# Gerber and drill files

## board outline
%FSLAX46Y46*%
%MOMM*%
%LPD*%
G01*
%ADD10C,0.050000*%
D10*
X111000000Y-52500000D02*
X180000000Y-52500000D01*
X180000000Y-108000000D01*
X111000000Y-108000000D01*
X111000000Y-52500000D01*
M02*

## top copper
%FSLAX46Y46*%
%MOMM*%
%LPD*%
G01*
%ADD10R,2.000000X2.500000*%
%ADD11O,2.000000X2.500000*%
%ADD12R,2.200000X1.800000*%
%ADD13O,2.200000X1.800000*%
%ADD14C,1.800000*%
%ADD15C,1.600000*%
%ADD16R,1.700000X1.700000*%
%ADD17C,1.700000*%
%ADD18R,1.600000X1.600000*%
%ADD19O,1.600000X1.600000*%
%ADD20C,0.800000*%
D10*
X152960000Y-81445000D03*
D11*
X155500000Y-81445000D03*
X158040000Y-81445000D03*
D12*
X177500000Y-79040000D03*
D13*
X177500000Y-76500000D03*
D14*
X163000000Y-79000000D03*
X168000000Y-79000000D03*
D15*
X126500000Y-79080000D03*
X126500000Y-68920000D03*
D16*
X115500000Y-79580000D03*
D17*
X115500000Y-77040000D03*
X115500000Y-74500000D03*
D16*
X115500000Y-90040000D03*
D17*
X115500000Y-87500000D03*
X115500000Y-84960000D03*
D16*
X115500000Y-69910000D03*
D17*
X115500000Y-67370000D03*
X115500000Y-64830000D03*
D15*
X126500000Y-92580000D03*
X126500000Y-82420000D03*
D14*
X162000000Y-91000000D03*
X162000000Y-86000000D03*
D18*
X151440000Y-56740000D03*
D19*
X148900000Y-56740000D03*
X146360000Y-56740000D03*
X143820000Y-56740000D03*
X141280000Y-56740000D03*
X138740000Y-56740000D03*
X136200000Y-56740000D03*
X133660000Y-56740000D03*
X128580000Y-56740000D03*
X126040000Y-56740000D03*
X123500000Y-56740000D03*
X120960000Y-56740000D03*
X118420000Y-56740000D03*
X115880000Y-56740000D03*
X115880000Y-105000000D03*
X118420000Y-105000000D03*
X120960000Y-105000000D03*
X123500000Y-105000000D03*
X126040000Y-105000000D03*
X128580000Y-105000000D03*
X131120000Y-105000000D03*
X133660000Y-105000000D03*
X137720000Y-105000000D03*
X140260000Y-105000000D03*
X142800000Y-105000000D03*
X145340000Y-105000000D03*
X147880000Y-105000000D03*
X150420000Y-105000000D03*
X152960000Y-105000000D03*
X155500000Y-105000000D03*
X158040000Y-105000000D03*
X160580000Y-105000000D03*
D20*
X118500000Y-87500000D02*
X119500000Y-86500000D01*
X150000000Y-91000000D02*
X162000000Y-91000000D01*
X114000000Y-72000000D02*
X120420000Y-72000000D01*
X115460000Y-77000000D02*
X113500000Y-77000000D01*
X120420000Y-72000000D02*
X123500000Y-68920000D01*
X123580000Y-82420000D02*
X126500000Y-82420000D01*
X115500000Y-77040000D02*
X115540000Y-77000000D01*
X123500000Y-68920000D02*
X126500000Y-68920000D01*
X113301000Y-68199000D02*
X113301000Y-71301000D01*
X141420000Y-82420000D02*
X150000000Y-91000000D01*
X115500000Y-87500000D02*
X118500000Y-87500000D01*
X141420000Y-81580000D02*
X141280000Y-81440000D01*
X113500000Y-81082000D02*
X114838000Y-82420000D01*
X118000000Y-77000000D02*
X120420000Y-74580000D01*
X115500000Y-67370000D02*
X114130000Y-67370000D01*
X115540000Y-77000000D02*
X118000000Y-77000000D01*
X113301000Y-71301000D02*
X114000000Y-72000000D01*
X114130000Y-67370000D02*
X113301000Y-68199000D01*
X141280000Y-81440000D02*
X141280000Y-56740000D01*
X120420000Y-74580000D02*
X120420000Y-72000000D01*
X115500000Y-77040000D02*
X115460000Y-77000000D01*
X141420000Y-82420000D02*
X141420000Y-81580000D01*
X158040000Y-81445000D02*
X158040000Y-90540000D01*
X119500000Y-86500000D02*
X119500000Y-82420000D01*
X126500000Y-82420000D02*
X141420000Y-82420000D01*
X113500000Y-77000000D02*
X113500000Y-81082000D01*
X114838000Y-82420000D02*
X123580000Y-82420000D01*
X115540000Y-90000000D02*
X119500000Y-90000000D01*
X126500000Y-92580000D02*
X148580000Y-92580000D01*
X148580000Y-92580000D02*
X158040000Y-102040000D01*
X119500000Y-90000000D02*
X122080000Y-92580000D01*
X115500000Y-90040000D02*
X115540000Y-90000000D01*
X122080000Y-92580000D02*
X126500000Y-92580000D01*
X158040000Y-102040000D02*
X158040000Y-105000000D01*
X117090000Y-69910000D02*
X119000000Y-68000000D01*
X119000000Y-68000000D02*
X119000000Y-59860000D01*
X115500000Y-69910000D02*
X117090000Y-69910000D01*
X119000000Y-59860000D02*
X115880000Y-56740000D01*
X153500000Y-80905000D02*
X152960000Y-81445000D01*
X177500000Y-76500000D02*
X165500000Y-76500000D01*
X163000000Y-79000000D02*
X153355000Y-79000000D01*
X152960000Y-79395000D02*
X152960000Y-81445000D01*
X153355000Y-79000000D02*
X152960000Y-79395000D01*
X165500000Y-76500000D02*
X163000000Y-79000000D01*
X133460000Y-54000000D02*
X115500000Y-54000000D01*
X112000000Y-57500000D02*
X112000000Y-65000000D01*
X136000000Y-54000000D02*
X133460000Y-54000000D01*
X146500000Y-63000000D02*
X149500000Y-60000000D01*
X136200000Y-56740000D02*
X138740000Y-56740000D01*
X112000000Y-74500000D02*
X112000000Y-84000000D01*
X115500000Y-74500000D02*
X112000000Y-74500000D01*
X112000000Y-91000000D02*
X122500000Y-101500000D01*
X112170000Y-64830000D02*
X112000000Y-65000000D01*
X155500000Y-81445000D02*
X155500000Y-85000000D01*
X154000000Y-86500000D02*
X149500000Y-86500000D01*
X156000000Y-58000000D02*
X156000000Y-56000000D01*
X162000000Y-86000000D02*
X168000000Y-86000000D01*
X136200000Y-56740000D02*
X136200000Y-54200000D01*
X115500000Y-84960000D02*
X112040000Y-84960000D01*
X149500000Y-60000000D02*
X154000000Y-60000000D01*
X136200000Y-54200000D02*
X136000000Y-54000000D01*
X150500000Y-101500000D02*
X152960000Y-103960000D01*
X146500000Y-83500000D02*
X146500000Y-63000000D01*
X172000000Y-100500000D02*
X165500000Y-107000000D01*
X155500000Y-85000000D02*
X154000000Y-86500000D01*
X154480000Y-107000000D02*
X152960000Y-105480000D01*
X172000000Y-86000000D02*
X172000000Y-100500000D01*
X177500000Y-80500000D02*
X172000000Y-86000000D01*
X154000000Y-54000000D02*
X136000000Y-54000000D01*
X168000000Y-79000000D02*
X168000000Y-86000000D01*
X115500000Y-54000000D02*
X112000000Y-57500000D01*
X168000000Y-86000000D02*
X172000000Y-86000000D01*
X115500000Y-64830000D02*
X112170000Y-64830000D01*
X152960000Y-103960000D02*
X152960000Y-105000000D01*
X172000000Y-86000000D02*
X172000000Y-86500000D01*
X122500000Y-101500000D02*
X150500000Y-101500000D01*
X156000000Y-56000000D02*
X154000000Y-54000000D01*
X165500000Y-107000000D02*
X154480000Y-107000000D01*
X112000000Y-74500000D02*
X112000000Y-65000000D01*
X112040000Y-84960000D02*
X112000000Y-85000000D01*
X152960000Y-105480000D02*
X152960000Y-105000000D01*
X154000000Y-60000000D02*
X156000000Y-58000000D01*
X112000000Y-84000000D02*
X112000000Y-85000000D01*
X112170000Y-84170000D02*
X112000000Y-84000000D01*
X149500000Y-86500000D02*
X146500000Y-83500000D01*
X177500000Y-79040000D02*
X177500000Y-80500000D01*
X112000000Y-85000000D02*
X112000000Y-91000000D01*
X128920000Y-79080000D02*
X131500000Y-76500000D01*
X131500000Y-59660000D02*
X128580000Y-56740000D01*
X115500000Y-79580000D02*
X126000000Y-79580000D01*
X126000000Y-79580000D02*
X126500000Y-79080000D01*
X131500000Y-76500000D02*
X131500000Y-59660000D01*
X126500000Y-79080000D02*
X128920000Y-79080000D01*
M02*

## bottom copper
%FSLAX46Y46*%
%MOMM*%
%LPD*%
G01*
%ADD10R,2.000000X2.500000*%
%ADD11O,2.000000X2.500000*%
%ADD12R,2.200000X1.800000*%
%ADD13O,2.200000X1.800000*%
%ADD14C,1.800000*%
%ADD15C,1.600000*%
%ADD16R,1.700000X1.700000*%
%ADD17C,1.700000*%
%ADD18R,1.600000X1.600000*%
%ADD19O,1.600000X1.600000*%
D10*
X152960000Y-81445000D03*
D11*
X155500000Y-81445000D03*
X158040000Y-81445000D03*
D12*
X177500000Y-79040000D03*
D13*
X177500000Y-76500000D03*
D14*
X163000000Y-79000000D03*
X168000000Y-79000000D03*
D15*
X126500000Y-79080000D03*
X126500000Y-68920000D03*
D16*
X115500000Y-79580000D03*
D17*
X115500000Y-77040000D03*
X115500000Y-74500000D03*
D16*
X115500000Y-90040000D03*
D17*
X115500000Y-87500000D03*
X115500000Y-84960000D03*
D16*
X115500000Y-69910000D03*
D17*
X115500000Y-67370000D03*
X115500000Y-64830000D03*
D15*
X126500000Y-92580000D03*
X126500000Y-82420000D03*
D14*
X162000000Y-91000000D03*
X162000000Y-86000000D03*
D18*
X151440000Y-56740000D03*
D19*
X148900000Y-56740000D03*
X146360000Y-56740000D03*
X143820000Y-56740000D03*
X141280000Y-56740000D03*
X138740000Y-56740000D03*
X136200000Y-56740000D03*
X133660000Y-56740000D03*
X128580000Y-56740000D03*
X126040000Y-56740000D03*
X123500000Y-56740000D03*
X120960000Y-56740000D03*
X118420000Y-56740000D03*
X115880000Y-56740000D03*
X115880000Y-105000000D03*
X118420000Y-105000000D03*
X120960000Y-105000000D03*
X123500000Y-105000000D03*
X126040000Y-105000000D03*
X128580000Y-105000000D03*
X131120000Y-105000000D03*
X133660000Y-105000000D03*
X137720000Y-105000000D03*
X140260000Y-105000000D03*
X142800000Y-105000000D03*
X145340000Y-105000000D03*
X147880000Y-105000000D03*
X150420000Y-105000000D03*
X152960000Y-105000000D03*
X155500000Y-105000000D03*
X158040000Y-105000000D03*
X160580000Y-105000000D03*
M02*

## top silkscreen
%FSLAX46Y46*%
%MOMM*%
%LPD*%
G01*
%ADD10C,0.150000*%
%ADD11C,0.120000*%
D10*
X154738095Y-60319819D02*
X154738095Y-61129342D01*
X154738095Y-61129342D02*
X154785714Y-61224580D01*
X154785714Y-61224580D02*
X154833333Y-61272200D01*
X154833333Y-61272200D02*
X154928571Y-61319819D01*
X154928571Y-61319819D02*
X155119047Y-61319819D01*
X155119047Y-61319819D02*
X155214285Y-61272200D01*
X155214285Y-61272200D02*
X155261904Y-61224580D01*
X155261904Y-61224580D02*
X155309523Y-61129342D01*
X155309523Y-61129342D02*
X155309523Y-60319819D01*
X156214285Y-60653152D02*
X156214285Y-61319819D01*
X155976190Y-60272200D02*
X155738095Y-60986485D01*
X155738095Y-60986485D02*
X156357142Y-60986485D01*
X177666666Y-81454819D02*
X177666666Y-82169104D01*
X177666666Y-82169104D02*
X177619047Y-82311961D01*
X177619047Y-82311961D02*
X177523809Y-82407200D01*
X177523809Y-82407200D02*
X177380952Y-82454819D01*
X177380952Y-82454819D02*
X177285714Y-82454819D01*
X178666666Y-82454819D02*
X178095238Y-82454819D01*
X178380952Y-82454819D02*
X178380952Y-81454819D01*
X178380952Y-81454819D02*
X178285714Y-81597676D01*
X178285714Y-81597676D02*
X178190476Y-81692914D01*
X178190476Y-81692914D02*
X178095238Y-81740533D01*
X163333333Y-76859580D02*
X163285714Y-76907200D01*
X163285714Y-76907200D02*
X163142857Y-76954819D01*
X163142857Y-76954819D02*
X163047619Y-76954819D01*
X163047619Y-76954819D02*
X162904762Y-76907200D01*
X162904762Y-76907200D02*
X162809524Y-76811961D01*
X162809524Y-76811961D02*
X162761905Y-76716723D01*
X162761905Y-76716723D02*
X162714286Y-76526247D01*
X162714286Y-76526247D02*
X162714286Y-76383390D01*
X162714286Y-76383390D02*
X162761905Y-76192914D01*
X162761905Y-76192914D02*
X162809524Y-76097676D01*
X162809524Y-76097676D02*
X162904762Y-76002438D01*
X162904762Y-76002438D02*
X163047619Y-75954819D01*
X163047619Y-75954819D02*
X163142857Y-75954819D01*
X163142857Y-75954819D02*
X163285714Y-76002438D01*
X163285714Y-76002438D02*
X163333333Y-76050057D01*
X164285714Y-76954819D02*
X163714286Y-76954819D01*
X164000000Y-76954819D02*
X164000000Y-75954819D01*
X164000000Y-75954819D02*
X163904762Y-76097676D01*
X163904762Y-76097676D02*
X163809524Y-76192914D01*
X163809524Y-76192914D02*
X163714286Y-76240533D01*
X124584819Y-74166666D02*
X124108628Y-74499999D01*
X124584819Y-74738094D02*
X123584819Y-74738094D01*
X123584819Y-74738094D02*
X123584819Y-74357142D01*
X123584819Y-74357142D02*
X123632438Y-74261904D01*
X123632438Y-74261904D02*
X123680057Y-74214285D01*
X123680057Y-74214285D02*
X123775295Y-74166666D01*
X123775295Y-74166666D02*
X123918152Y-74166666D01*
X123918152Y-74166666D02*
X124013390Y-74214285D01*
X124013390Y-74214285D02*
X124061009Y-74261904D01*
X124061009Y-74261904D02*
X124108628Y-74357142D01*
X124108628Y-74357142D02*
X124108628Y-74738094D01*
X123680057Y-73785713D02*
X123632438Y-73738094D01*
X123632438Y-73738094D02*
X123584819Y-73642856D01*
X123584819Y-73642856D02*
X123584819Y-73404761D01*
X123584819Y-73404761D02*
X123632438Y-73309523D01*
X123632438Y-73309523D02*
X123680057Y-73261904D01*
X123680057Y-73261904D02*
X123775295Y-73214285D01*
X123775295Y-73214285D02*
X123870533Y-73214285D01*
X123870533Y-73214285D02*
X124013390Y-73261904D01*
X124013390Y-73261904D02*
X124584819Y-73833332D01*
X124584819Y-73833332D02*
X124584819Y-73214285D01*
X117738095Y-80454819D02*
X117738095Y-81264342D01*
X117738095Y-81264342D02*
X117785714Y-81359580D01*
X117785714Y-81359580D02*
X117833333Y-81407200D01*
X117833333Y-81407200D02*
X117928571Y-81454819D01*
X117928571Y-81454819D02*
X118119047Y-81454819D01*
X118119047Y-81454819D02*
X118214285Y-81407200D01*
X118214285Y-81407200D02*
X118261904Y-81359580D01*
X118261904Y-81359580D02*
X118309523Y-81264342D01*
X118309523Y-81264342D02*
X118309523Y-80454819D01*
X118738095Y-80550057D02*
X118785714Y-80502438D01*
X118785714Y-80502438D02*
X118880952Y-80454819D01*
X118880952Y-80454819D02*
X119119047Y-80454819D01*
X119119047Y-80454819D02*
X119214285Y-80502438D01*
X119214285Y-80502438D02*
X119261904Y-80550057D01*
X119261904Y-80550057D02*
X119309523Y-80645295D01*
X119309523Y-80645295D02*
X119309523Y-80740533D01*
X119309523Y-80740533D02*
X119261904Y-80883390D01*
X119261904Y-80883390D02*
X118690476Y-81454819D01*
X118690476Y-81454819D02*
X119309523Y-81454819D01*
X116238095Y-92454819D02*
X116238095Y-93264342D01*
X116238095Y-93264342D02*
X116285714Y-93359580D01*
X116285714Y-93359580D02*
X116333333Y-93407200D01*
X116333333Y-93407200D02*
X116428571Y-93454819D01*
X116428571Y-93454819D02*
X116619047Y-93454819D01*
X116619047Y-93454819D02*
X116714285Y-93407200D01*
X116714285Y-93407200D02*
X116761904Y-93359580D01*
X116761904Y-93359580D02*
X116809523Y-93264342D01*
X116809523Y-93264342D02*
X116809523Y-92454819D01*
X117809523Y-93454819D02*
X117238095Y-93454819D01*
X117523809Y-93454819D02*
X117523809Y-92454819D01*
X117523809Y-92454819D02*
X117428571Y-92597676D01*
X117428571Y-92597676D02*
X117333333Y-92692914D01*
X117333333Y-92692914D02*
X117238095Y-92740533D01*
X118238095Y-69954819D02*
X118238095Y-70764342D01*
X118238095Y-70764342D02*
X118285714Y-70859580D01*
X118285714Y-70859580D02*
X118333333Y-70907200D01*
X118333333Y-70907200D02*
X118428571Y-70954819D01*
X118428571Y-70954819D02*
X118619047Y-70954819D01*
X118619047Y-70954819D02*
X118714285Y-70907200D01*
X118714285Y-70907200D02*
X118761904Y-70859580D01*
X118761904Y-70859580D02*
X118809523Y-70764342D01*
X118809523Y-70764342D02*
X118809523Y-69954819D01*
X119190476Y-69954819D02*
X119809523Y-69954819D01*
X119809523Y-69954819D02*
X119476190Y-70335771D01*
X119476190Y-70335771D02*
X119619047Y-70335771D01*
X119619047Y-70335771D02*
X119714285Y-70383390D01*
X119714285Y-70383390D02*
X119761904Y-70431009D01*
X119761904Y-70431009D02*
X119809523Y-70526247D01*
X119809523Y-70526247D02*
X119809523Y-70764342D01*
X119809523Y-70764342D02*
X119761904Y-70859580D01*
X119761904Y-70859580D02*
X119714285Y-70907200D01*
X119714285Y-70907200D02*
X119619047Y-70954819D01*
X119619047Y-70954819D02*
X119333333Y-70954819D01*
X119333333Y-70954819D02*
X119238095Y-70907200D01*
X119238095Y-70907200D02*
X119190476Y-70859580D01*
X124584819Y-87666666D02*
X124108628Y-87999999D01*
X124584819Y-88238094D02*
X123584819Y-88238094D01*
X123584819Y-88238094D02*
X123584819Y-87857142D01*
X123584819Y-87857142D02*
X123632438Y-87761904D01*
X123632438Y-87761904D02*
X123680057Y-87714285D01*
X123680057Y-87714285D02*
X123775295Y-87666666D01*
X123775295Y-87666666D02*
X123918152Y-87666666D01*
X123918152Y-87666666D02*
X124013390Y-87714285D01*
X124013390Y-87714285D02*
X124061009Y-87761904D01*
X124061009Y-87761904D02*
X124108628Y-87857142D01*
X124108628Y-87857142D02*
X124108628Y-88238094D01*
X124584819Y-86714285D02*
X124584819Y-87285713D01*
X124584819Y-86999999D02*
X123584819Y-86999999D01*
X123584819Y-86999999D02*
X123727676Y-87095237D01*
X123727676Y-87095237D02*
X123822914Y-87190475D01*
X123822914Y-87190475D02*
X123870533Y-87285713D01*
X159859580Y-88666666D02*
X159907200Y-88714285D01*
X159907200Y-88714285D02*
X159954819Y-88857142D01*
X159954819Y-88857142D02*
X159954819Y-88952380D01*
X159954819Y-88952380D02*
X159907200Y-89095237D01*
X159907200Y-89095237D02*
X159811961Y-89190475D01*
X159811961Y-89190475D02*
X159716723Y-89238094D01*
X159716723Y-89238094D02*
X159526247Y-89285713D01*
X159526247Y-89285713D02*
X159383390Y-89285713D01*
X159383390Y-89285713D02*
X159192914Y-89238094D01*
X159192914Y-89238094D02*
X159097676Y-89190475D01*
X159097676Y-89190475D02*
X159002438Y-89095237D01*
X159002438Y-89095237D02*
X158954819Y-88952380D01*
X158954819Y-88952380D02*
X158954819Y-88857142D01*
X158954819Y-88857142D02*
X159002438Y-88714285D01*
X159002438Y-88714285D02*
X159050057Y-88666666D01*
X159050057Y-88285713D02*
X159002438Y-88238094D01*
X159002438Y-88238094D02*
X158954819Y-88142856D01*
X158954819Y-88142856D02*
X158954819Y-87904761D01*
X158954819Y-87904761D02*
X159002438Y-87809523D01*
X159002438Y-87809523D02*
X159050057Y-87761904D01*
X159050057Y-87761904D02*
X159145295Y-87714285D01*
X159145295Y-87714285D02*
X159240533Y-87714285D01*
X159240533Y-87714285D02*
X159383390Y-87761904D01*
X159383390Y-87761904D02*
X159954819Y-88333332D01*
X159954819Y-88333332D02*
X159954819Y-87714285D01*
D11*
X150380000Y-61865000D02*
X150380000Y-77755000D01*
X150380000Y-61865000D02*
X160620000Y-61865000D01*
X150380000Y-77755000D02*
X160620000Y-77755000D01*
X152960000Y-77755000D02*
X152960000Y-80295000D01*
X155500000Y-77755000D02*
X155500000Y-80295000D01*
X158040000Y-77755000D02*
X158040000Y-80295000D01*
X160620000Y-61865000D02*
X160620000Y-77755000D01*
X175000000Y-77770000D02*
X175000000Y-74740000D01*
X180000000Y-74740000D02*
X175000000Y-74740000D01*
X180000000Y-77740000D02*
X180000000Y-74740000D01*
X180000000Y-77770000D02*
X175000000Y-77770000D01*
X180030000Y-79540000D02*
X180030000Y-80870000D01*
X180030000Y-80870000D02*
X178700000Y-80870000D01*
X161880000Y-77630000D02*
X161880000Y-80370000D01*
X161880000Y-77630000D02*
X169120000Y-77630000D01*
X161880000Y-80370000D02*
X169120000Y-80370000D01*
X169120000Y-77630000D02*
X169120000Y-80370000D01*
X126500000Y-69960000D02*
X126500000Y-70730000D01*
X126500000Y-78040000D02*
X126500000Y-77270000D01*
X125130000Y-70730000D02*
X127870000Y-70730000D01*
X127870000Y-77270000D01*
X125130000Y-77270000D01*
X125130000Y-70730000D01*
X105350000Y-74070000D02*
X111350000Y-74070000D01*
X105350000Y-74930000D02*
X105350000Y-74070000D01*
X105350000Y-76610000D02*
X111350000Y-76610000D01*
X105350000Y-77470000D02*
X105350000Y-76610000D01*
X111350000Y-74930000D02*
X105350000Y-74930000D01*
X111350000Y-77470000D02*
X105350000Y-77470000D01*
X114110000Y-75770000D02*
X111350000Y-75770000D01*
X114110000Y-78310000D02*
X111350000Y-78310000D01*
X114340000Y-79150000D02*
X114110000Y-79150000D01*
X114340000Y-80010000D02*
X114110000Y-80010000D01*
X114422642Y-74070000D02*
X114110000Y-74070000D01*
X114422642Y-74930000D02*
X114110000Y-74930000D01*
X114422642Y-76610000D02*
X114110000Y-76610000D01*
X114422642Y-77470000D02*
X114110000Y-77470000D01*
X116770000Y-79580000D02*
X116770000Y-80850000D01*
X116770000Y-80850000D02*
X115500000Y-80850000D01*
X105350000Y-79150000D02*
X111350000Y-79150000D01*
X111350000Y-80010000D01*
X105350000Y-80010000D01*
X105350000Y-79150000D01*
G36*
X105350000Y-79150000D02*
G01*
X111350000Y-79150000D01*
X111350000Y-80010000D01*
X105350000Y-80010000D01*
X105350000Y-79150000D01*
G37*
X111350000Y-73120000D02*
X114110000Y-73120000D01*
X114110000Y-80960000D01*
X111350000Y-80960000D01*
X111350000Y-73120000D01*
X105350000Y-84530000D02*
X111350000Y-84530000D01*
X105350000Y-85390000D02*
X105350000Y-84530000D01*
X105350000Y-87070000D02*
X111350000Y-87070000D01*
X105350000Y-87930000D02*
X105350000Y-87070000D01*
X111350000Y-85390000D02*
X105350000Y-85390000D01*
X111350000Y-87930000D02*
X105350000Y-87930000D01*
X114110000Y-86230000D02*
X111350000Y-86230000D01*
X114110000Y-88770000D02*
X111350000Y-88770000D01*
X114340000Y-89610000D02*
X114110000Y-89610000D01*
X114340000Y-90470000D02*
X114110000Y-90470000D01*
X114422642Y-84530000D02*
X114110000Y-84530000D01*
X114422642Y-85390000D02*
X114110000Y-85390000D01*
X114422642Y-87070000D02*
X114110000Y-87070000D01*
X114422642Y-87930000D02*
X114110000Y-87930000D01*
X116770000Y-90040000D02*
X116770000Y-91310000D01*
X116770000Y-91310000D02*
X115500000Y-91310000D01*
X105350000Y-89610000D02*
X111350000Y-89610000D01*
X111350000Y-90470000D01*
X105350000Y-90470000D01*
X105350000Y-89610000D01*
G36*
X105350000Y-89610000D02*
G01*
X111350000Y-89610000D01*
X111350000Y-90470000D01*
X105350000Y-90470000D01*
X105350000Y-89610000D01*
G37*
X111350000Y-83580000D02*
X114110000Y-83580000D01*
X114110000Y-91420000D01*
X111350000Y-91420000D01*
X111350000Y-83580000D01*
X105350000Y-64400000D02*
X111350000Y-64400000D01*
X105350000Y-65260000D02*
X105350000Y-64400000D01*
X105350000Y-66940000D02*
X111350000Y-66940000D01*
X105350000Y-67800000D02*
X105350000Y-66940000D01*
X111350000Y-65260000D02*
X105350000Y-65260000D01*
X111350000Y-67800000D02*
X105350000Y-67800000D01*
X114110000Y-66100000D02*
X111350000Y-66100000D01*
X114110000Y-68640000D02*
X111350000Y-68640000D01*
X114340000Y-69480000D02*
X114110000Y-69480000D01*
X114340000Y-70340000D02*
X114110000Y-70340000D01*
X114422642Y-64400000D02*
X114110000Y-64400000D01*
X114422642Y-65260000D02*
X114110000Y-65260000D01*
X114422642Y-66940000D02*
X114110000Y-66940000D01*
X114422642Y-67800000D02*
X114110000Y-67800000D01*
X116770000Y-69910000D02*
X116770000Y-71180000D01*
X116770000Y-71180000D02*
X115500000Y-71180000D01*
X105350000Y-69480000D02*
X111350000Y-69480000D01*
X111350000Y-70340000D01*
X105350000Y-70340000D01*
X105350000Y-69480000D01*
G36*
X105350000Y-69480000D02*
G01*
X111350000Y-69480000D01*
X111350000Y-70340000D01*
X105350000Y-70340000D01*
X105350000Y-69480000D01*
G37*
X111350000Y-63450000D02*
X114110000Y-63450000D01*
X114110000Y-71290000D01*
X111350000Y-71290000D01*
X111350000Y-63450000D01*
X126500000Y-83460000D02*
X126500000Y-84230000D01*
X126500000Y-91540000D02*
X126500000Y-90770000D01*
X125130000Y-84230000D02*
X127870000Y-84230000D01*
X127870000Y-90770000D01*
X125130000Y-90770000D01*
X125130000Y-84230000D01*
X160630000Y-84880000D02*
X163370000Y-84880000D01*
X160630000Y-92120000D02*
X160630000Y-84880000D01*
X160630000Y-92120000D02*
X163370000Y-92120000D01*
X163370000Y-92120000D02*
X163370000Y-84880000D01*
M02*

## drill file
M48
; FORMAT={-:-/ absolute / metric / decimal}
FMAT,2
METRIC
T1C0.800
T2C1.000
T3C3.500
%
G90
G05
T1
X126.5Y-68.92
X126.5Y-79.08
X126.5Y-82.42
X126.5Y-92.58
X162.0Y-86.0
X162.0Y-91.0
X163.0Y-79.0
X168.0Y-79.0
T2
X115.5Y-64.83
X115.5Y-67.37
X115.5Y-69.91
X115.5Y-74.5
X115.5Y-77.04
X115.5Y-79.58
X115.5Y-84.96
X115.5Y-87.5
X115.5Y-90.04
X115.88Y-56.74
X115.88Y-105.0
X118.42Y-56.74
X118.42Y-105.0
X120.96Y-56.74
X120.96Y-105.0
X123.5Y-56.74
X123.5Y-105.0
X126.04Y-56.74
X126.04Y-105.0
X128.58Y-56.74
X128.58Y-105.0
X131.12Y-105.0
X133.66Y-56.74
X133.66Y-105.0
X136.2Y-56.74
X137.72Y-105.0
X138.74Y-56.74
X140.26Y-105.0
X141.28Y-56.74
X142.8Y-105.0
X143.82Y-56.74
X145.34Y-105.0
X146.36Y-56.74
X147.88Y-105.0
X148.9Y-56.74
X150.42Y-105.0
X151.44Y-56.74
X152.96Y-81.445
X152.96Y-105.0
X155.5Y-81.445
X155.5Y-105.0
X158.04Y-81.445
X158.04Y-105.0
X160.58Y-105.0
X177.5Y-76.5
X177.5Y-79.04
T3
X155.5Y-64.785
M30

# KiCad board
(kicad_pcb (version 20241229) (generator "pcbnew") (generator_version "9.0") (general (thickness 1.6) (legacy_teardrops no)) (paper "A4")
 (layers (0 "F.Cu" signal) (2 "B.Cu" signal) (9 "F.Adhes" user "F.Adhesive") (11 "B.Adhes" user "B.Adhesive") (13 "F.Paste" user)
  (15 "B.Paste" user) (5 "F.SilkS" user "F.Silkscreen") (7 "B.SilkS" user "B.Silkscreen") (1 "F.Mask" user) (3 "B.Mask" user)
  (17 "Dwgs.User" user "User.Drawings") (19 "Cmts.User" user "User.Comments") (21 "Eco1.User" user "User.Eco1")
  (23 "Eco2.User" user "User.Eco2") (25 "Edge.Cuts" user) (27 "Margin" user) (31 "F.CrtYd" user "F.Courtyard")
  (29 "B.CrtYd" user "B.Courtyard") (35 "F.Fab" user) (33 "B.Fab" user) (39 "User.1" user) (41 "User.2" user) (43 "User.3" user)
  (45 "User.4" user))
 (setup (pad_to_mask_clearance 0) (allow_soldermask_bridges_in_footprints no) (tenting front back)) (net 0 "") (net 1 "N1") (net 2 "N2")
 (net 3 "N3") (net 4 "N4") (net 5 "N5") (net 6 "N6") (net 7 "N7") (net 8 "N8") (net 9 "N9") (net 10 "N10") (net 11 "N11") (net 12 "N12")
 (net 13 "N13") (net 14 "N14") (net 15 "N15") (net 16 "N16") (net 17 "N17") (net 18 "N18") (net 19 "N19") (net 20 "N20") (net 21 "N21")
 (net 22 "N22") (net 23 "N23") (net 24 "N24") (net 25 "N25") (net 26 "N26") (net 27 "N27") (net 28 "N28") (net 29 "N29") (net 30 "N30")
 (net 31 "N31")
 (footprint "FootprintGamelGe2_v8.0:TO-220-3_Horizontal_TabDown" (layer "F.Cu") (at 152.96 81.445)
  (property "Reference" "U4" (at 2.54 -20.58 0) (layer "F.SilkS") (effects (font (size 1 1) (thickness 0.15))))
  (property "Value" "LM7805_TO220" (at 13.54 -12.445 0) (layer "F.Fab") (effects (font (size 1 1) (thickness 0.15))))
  (fp_line (start -2.58 -19.58) (end -2.58 -3.69) (stroke (width 0.12) (type solid)) (layer "F.SilkS"))
  (fp_line (start -2.58 -19.58) (end 7.66 -19.58) (stroke (width 0.12) (type solid)) (layer "F.SilkS"))
  (fp_line (start -2.58 -3.69) (end 7.66 -3.69) (stroke (width 0.12) (type solid)) (layer "F.SilkS"))
  (fp_line (start 0 -3.69) (end 0 -1.15) (stroke (width 0.12) (type solid)) (layer "F.SilkS"))
  (fp_line (start 2.54 -3.69) (end 2.54 -1.15) (stroke (width 0.12) (type solid)) (layer "F.SilkS"))
  (fp_line (start 5.08 -3.69) (end 5.08 -1.15) (stroke (width 0.12) (type solid)) (layer "F.SilkS"))
  (fp_line (start 7.66 -19.58) (end 7.66 -3.69) (stroke (width 0.12) (type solid)) (layer "F.SilkS"))
  (pad "" np_thru_hole oval (at 2.54 -16.66) (size 3.5 3.5) (drill 3.5) (layers "*.Cu" "*.Mask"))
  (pad "1" thru_hole rect (at 0 0) (size 2 2.5) (drill 1) (layers "*.Cu" "*.Mask") (remove_unused_layers no) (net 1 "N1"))
  (pad "2" thru_hole oval (at 2.54 0) (size 2 2.5) (drill 1) (layers "*.Cu" "*.Mask") (remove_unused_layers no) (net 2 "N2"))
  (pad "3" thru_hole oval (at 5.08 0) (size 2 2.5) (drill 1) (layers "*.Cu" "*.Mask") (remove_unused_layers no) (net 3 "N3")))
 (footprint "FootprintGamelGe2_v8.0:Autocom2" (layer "F.Cu") (at 177.5 79.04 180)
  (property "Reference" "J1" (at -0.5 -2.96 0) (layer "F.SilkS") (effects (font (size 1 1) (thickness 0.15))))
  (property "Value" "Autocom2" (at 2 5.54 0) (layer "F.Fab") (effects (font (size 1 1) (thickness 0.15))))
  (fp_line (start 2.5 1.27) (end 2.5 4.3) (stroke (width 0.12) (type solid)) (layer "F.SilkS"))
  (fp_line (start -2.5 4.3) (end 2.5 4.3) (stroke (width 0.12) (type solid)) (layer "F.SilkS"))
  (fp_line (start -2.5 1.3) (end -2.5 4.3) (stroke (width 0.12) (type solid)) (layer "F.SilkS"))
  (fp_line (start -2.5 1.27) (end 2.5 1.27) (stroke (width 0.12) (type solid)) (layer "F.SilkS"))
  (fp_line (start -2.53 -0.5) (end -2.53 -1.83) (stroke (width 0.12) (type solid)) (layer "F.SilkS"))
  (fp_line (start -2.53 -1.83) (end -1.2 -1.83) (stroke (width 0.12) (type solid)) (layer "F.SilkS"))
  (pad "1" thru_hole rect (at 0 0 180) (size 2.2 1.8) (drill 1) (layers "*.Cu" "*.Mask") (remove_unused_layers no) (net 2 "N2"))
  (pad "2" thru_hole oval (at 0 2.54 180) (size 2.2 1.8) (drill 1) (layers "*.Cu" "*.Mask") (remove_unused_layers no) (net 1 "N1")))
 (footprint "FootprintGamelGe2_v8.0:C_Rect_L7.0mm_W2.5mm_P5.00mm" (layer "F.Cu") (at 163 79)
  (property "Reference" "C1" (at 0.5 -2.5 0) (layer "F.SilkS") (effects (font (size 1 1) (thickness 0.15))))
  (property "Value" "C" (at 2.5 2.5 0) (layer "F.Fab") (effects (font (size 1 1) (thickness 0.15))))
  (fp_line (start -1.12 -1.37) (end -1.12 1.37) (stroke (width 0.12) (type solid)) (layer "F.SilkS"))
  (fp_line (start -1.12 -1.37) (end 6.12 -1.37) (stroke (width 0.12) (type solid)) (layer "F.SilkS"))
  (fp_line (start -1.12 1.37) (end 6.12 1.37) (stroke (width 0.12) (type solid)) (layer "F.SilkS"))
  (fp_line (start 6.12 -1.37) (end 6.12 1.37) (stroke (width 0.12) (type solid)) (layer "F.SilkS"))
  (pad "1" thru_hole circle (at 0 0) (size 1.8 1.8) (drill 0.8) (layers "*.Cu" "*.Mask") (remove_unused_layers no) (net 1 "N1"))
  (pad "2" thru_hole circle (at 5 0) (size 1.8 1.8) (drill 0.8) (layers "*.Cu" "*.Mask") (remove_unused_layers no) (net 2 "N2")))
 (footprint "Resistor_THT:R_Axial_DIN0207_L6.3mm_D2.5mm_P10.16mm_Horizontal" (layer "F.Cu") (at 126.5 79.08 90)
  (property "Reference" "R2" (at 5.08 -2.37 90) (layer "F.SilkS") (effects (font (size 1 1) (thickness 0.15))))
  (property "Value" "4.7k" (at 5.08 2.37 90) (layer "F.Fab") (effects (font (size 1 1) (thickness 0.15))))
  (fp_line (start 9.12 0) (end 8.35 0) (stroke (width 0.12) (type solid)) (layer "F.SilkS"))
  (fp_line (start 1.04 0) (end 1.81 0) (stroke (width 0.12) (type solid)) (layer "F.SilkS"))
  (fp_rect (start 1.81 -1.37) (end 8.35 1.37) (stroke (width 0.12) (type solid)) (fill no) (layer "F.SilkS"))
  (pad "1" thru_hole circle (at 0 0 90) (size 1.6 1.6) (drill 0.8) (layers "*.Cu" "*.Mask") (remove_unused_layers no) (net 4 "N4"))
  (pad "2" thru_hole circle (at 10.16 0 90) (size 1.6 1.6) (drill 0.8) (layers "*.Cu" "*.Mask") (remove_unused_layers no) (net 3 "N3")))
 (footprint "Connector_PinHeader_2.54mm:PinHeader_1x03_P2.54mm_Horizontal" (layer "F.Cu") (at 115.5 79.58 180)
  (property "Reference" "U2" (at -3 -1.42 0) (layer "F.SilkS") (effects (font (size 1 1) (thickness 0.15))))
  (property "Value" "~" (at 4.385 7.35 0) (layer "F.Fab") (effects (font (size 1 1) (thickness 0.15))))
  (fp_line (start 10.15 5.51) (end 4.15 5.51) (stroke (width 0.12) (type solid)) (layer "F.SilkS"))
  (fp_line (start 10.15 4.65) (end 10.15 5.51) (stroke (width 0.12) (type solid)) (layer "F.SilkS"))
  (fp_line (start 10.15 2.97) (end 4.15 2.97) (stroke (width 0.12) (type solid)) (layer "F.SilkS"))
  (fp_line (start 10.15 2.11) (end 10.15 2.97) (stroke (width 0.12) (type solid)) (layer "F.SilkS"))
  (fp_line (start 4.15 4.65) (end 10.15 4.65) (stroke (width 0.12) (type solid)) (layer "F.SilkS"))
  (fp_line (start 4.15 2.11) (end 10.15 2.11) (stroke (width 0.12) (type solid)) (layer "F.SilkS"))
  (fp_line (start 1.39 3.81) (end 4.15 3.81) (stroke (width 0.12) (type solid)) (layer "F.SilkS"))
  (fp_line (start 1.39 1.27) (end 4.15 1.27) (stroke (width 0.12) (type solid)) (layer "F.SilkS"))
  (fp_line (start 1.16 0.43) (end 1.39 0.43) (stroke (width 0.12) (type solid)) (layer "F.SilkS"))
  (fp_line (start 1.16 -0.43) (end 1.39 -0.43) (stroke (width 0.12) (type solid)) (layer "F.SilkS"))
  (fp_line (start 1.077358 5.51) (end 1.39 5.51) (stroke (width 0.12) (type solid)) (layer "F.SilkS"))
  (fp_line (start 1.077358 4.65) (end 1.39 4.65) (stroke (width 0.12) (type solid)) (layer "F.SilkS"))
  (fp_line (start 1.077358 2.97) (end 1.39 2.97) (stroke (width 0.12) (type solid)) (layer "F.SilkS"))
  (fp_line (start 1.077358 2.11) (end 1.39 2.11) (stroke (width 0.12) (type solid)) (layer "F.SilkS"))
  (fp_line (start -1.27 0) (end -1.27 -1.27) (stroke (width 0.12) (type solid)) (layer "F.SilkS"))
  (fp_line (start -1.27 -1.27) (end 0 -1.27) (stroke (width 0.12) (type solid)) (layer "F.SilkS"))
  (fp_rect (start 4.15 -0.43) (end 10.15 0.43) (stroke (width 0.12) (type solid)) (fill yes) (layer "F.SilkS"))
  (fp_rect (start 1.39 -1.38) (end 4.15 6.46) (stroke (width 0.12) (type solid)) (fill no) (layer "F.SilkS"))
  (pad "1" thru_hole rect (at 0 0 180) (size 1.7 1.7) (drill 1) (layers "*.Cu" "*.Mask") (remove_unused_layers no) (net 4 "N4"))
  (pad "2" thru_hole circle (at 0 2.54 180) (size 1.7 1.7) (drill 1) (layers "*.Cu" "*.Mask") (remove_unused_layers no) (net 3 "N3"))
  (pad "3" thru_hole circle (at 0 5.08 180) (size 1.7 1.7) (drill 1) (layers "*.Cu" "*.Mask") (remove_unused_layers no) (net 2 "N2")))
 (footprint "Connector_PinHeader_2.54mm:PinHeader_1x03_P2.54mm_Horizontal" (layer "F.Cu") (at 115.5 90.04 180)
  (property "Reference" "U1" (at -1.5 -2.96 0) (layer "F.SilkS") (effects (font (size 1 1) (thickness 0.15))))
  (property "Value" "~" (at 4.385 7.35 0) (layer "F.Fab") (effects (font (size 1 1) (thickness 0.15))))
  (fp_line (start 10.15 5.51) (end 4.15 5.51) (stroke (width 0.12) (type solid)) (layer "F.SilkS"))
  (fp_line (start 10.15 4.65) (end 10.15 5.51) (stroke (width 0.12) (type solid)) (layer "F.SilkS"))
  (fp_line (start 10.15 2.97) (end 4.15 2.97) (stroke (width 0.12) (type solid)) (layer "F.SilkS"))
  (fp_line (start 10.15 2.11) (end 10.15 2.97) (stroke (width 0.12) (type solid)) (layer "F.SilkS"))
  (fp_line (start 4.15 4.65) (end 10.15 4.65) (stroke (width 0.12) (type solid)) (layer "F.SilkS"))
  (fp_line (start 4.15 2.11) (end 10.15 2.11) (stroke (width 0.12) (type solid)) (layer "F.SilkS"))
  (fp_line (start 1.39 3.81) (end 4.15 3.81) (stroke (width 0.12) (type solid)) (layer "F.SilkS"))
  (fp_line (start 1.39 1.27) (end 4.15 1.27) (stroke (width 0.12) (type solid)) (layer "F.SilkS"))
  (fp_line (start 1.16 0.43) (end 1.39 0.43) (stroke (width 0.12) (type solid)) (layer "F.SilkS"))
  (fp_line (start 1.16 -0.43) (end 1.39 -0.43) (stroke (width 0.12) (type solid)) (layer "F.SilkS"))
  (fp_line (start 1.077358 5.51) (end 1.39 5.51) (stroke (width 0.12) (type solid)) (layer "F.SilkS"))
  (fp_line (start 1.077358 4.65) (end 1.39 4.65) (stroke (width 0.12) (type solid)) (layer "F.SilkS"))
  (fp_line (start 1.077358 2.97) (end 1.39 2.97) (stroke (width 0.12) (type solid)) (layer "F.SilkS"))
  (fp_line (start 1.077358 2.11) (end 1.39 2.11) (stroke (width 0.12) (type solid)) (layer "F.SilkS"))
  (fp_line (start -1.27 0) (end -1.27 -1.27) (stroke (width 0.12) (type solid)) (layer "F.SilkS"))
  (fp_line (start -1.27 -1.27) (end 0 -1.27) (stroke (width 0.12) (type solid)) (layer "F.SilkS"))
  (fp_rect (start 4.15 -0.43) (end 10.15 0.43) (stroke (width 0.12) (type solid)) (fill yes) (layer "F.SilkS"))
  (fp_rect (start 1.39 -1.38) (end 4.15 6.46) (stroke (width 0.12) (type solid)) (fill no) (layer "F.SilkS"))
  (pad "1" thru_hole rect (at 0 0 180) (size 1.7 1.7) (drill 1) (layers "*.Cu" "*.Mask") (remove_unused_layers no) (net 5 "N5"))
  (pad "2" thru_hole circle (at 0 2.54 180) (size 1.7 1.7) (drill 1) (layers "*.Cu" "*.Mask") (remove_unused_layers no) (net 3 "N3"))
  (pad "3" thru_hole circle (at 0 5.08 180) (size 1.7 1.7) (drill 1) (layers "*.Cu" "*.Mask") (remove_unused_layers no) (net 2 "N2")))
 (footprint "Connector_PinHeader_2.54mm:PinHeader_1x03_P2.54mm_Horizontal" (layer "F.Cu") (at 115.5 69.91 180)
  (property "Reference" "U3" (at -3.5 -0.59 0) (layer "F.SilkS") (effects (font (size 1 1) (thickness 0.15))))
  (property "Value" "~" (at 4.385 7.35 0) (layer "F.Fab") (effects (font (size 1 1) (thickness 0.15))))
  (fp_line (start 10.15 5.51) (end 4.15 5.51) (stroke (width 0.12) (type solid)) (layer "F.SilkS"))
  (fp_line (start 10.15 4.65) (end 10.15 5.51) (stroke (width 0.12) (type solid)) (layer "F.SilkS"))
  (fp_line (start 10.15 2.97) (end 4.15 2.97) (stroke (width 0.12) (type solid)) (layer "F.SilkS"))
  (fp_line (start 10.15 2.11) (end 10.15 2.97) (stroke (width 0.12) (type solid)) (layer "F.SilkS"))
  (fp_line (start 4.15 4.65) (end 10.15 4.65) (stroke (width 0.12) (type solid)) (layer "F.SilkS"))
  (fp_line (start 4.15 2.11) (end 10.15 2.11) (stroke (width 0.12) (type solid)) (layer "F.SilkS"))
  (fp_line (start 1.39 3.81) (end 4.15 3.81) (stroke (width 0.12) (type solid)) (layer "F.SilkS"))
  (fp_line (start 1.39 1.27) (end 4.15 1.27) (stroke (width 0.12) (type solid)) (layer "F.SilkS"))
  (fp_line (start 1.16 0.43) (end 1.39 0.43) (stroke (width 0.12) (type solid)) (layer "F.SilkS"))
  (fp_line (start 1.16 -0.43) (end 1.39 -0.43) (stroke (width 0.12) (type solid)) (layer "F.SilkS"))
  (fp_line (start 1.077358 5.51) (end 1.39 5.51) (stroke (width 0.12) (type solid)) (layer "F.SilkS"))
  (fp_line (start 1.077358 4.65) (end 1.39 4.65) (stroke (width 0.12) (type solid)) (layer "F.SilkS"))
  (fp_line (start 1.077358 2.97) (end 1.39 2.97) (stroke (width 0.12) (type solid)) (layer "F.SilkS"))
  (fp_line (start 1.077358 2.11) (end 1.39 2.11) (stroke (width 0.12) (type solid)) (layer "F.SilkS"))
  (fp_line (start -1.27 0) (end -1.27 -1.27) (stroke (width 0.12) (type solid)) (layer "F.SilkS"))
  (fp_line (start -1.27 -1.27) (end 0 -1.27) (stroke (width 0.12) (type solid)) (layer "F.SilkS"))
  (fp_rect (start 4.15 -0.43) (end 10.15 0.43) (stroke (width 0.12) (type solid)) (fill yes) (layer "F.SilkS"))
  (fp_rect (start 1.39 -1.38) (end 4.15 6.46) (stroke (width 0.12) (type solid)) (fill no) (layer "F.SilkS"))
  (pad "1" thru_hole rect (at 0 0 180) (size 1.7 1.7) (drill 1) (layers "*.Cu" "*.Mask") (remove_unused_layers no) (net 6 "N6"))
  (pad "2" thru_hole circle (at 0 2.54 180) (size 1.7 1.7) (drill 1) (layers "*.Cu" "*.Mask") (remove_unused_layers no) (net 3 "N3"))
  (pad "3" thru_hole circle (at 0 5.08 180) (size 1.7 1.7) (drill 1) (layers "*.Cu" "*.Mask") (remove_unused_layers no) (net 2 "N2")))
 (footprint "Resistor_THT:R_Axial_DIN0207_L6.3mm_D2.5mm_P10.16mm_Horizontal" (layer "F.Cu") (at 126.5 92.58 90)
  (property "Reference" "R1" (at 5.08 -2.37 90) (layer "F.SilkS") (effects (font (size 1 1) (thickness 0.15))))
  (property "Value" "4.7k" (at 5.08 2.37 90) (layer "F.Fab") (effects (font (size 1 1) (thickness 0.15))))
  (fp_line (start 9.12 0) (end 8.35 0) (stroke (width 0.12) (type solid)) (layer "F.SilkS"))
  (fp_line (start 1.04 0) (end 1.81 0) (stroke (width 0.12) (type solid)) (layer "F.SilkS"))
  (fp_rect (start 1.81 -1.37) (end 8.35 1.37) (stroke (width 0.12) (type solid)) (fill no) (layer "F.SilkS"))
  (pad "1" thru_hole circle (at 0 0 90) (size 1.6 1.6) (drill 0.8) (layers "*.Cu" "*.Mask") (remove_unused_layers no) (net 5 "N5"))
  (pad "2" thru_hole circle (at 10.16 0 90) (size 1.6 1.6) (drill 0.8) (layers "*.Cu" "*.Mask") (remove_unused_layers no) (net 3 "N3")))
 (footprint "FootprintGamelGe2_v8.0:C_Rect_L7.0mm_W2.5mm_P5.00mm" (layer "F.Cu") (at 162 91 90)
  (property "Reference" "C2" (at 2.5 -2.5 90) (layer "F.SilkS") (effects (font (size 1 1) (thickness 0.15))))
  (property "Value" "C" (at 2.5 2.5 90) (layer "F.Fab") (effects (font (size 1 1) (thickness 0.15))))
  (fp_line (start 6.12 -1.37) (end 6.12 1.37) (stroke (width 0.12) (type solid)) (layer "F.SilkS"))
  (fp_line (start -1.12 -1.37) (end 6.12 -1.37) (stroke (width 0.12) (type solid)) (layer "F.SilkS"))
  (fp_line (start -1.12 -1.37) (end -1.12 1.37) (stroke (width 0.12) (type solid)) (layer "F.SilkS"))
  (fp_line (start -1.12 1.37) (end 6.12 1.37) (stroke (width 0.12) (type solid)) (layer "F.SilkS"))
  (pad "1" thru_hole circle (at 0 0 90) (size 1.8 1.8) (drill 0.8) (layers "*.Cu" "*.Mask") (remove_unused_layers no) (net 3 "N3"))
  (pad "2" thru_hole circle (at 5 0 90) (size 1.8 1.8) (drill 0.8) (layers "*.Cu" "*.Mask") (remove_unused_layers no) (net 2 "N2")))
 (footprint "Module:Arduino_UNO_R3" (layer "B.Cu") (at 151.44 56.74 180)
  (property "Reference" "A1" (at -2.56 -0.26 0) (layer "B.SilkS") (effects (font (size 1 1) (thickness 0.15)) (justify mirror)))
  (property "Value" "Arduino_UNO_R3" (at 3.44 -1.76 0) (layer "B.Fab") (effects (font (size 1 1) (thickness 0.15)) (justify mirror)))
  (pad "1" thru_hole rect (at 0 0 90) (size 1.6 1.6) (drill 1) (layers "*.Cu" "*.Mask") (remove_unused_layers no) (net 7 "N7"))
  (pad "2" thru_hole oval (at 2.54 0 90) (size 1.6 1.6) (drill 1) (layers "*.Cu" "*.Mask") (remove_unused_layers no) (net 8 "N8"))
  (pad "3" thru_hole oval (at 5.08 0 90) (size 1.6 1.6) (drill 1) (layers "*.Cu" "*.Mask") (remove_unused_layers no) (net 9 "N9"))
  (pad "4" thru_hole oval (at 7.62 0 90) (size 1.6 1.6) (drill 1) (layers "*.Cu" "*.Mask") (remove_unused_layers no) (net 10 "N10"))
  (pad "5" thru_hole oval (at 10.16 0 90) (size 1.6 1.6) (drill 1) (layers "*.Cu" "*.Mask") (remove_unused_layers no) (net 3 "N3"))
  (pad "6" thru_hole oval (at 12.7 0 90) (size 1.6 1.6) (drill 1) (layers "*.Cu" "*.Mask") (remove_unused_layers no) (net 2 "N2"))
  (pad "7" thru_hole oval (at 15.24 0 90) (size 1.6 1.6) (drill 1) (layers "*.Cu" "*.Mask") (remove_unused_layers no) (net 2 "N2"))
  (pad "8" thru_hole oval (at 17.78 0 90) (size 1.6 1.6) (drill 1) (layers "*.Cu" "*.Mask") (remove_unused_layers no) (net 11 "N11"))
  (pad "9" thru_hole oval (at 22.86 0 90) (size 1.6 1.6) (drill 1) (layers "*.Cu" "*.Mask") (remove_unused_layers no) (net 4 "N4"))
  (pad "10" thru_hole oval (at 25.4 0 90) (size 1.6 1.6) (drill 1) (layers "*.Cu" "*.Mask") (remove_unused_layers no) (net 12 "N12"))
  (pad "11" thru_hole oval (at 27.94 0 90) (size 1.6 1.6) (drill 1) (layers "*.Cu" "*.Mask") (remove_unused_layers no) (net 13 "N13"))
  (pad "12" thru_hole oval (at 30.48 0 90) (size 1.6 1.6) (drill 1) (layers "*.Cu" "*.Mask") (remove_unused_layers no) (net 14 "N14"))
  (pad "13" thru_hole oval (at 33.02 0 90) (size 1.6 1.6) (drill 1) (layers "*.Cu" "*.Mask") (remove_unused_layers no) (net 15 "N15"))
  (pad "14" thru_hole oval (at 35.56 0 90) (size 1.6 1.6) (drill 1) (layers "*.Cu" "*.Mask") (remove_unused_layers no) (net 6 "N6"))
  (pad "15" thru_hole oval (at 35.56 -48.26 90) (size 1.6 1.6) (drill 1) (layers "*.Cu" "*.Mask") (remove_unused_layers no) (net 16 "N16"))
  (pad "16" thru_hole oval (at 33.02 -48.26 90) (size 1.6 1.6) (drill 1) (layers "*.Cu" "*.Mask") (remove_unused_layers no) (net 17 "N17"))
  (pad "17" thru_hole oval (at 30.48 -48.26 90) (size 1.6 1.6) (drill 1) (layers "*.Cu" "*.Mask") (remove_unused_layers no) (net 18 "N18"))
  (pad "18" thru_hole oval (at 27.94 -48.26 90) (size 1.6 1.6) (drill 1) (layers "*.Cu" "*.Mask") (remove_unused_layers no) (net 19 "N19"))
  (pad "19" thru_hole oval (at 25.4 -48.26 90) (size 1.6 1.6) (drill 1) (layers "*.Cu" "*.Mask") (remove_unused_layers no) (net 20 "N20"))
  (pad "20" thru_hole oval (at 22.86 -48.26 90) (size 1.6 1.6) (drill 1) (layers "*.Cu" "*.Mask") (remove_unused_layers no) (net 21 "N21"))
  (pad "21" thru_hole oval (at 20.32 -48.26 90) (size 1.6 1.6) (drill 1) (layers "*.Cu" "*.Mask") (remove_unused_layers no) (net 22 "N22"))
  (pad "22" thru_hole oval (at 17.78 -48.26 90) (size 1.6 1.6) (drill 1) (layers "*.Cu" "*.Mask") (remove_unused_layers no) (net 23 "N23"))
  (pad "23" thru_hole oval (at 13.72 -48.26 90) (size 1.6 1.6) (drill 1) (layers "*.Cu" "*.Mask") (remove_unused_layers no) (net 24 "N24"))
  (pad "24" thru_hole oval (at 11.18 -48.26 90) (size 1.6 1.6) (drill 1) (layers "*.Cu" "*.Mask") (remove_unused_layers no) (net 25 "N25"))
  (pad "25" thru_hole oval (at 8.64 -48.26 90) (size 1.6 1.6) (drill 1) (layers "*.Cu" "*.Mask") (remove_unused_layers no) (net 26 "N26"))
  (pad "26" thru_hole oval (at 6.1 -48.26 90) (size 1.6 1.6) (drill 1) (layers "*.Cu" "*.Mask") (remove_unused_layers no) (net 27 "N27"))
  (pad "27" thru_hole oval (at 3.56 -48.26 90) (size 1.6 1.6) (drill 1) (layers "*.Cu" "*.Mask") (remove_unused_layers no) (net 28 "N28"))
  (pad "28" thru_hole oval (at 1.02 -48.26 90) (size 1.6 1.6) (drill 1) (layers "*.Cu" "*.Mask") (remove_unused_layers no) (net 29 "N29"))
  (pad "29" thru_hole oval (at -1.52 -48.26 90) (size 1.6 1.6) (drill 1) (layers "*.Cu" "*.Mask") (remove_unused_layers no) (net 2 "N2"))
  (pad "30" thru_hole oval (at -4.06 -48.26 90) (size 1.6 1.6) (drill 1) (layers "*.Cu" "*.Mask") (remove_unused_layers no) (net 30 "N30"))
  (pad "31" thru_hole oval (at -6.6 -48.26 90) (size 1.6 1.6) (drill 1) (layers "*.Cu" "*.Mask") (remove_unused_layers no) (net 5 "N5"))
  (pad "32" thru_hole oval (at -9.14 -48.26 90) (size 1.6 1.6) (drill 1) (layers "*.Cu" "*.Mask") (remove_unused_layers no) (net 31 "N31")))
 (gr_rect (start 111 52.5) (end 180 108) (stroke (width 0.05) (type default)) (fill no) (layer "Edge.Cuts"))
 (segment (start 118.5 87.5) (end 119.5 86.5) (width 0.8) (layer "F.Cu") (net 3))
 (segment (start 150 91) (end 162 91) (width 0.8) (layer "F.Cu") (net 3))
 (segment (start 114 72) (end 120.42 72) (width 0.8) (layer "F.Cu") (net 3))
 (segment (start 115.46 77) (end 113.5 77) (width 0.8) (layer "F.Cu") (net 3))
 (segment (start 120.42 72) (end 123.5 68.92) (width 0.8) (layer "F.Cu") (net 3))
 (segment (start 123.58 82.42) (end 126.5 82.42) (width 0.8) (layer "F.Cu") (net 3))
 (segment (start 115.5 77.04) (end 115.54 77) (width 0.8) (layer "F.Cu") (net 3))
 (segment (start 123.5 68.92) (end 126.5 68.92) (width 0.8) (layer "F.Cu") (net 3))
 (segment (start 113.301 68.199) (end 113.301 71.301) (width 0.8) (layer "F.Cu") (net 3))
 (segment (start 141.42 82.42) (end 150 91) (width 0.8) (layer "F.Cu") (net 3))
 (segment (start 115.5 87.5) (end 118.5 87.5) (width 0.8) (layer "F.Cu") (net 3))
 (segment (start 141.42 81.58) (end 141.28 81.44) (width 0.8) (layer "F.Cu") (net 3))
 (segment (start 113.5 81.082) (end 114.838 82.42) (width 0.8) (layer "F.Cu") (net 3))
 (segment (start 118 77) (end 120.42 74.58) (width 0.8) (layer "F.Cu") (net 3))
 (segment (start 115.5 67.37) (end 114.13 67.37) (width 0.8) (layer "F.Cu") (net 3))
 (segment (start 115.54 77) (end 118 77) (width 0.8) (layer "F.Cu") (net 3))
 (segment (start 113.301 71.301) (end 114 72) (width 0.8) (layer "F.Cu") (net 3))
 (segment (start 114.13 67.37) (end 113.301 68.199) (width 0.8) (layer "F.Cu") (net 3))
 (segment (start 141.28 81.44) (end 141.28 56.74) (width 0.8) (layer "F.Cu") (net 3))
 (segment (start 120.42 74.58) (end 120.42 72) (width 0.8) (layer "F.Cu") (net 3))
 (segment (start 115.5 77.04) (end 115.46 77) (width 0.8) (layer "F.Cu") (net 3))
 (segment (start 141.42 82.42) (end 141.42 81.58) (width 0.8) (layer "F.Cu") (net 3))
 (segment (start 158.04 81.445) (end 158.04 90.54) (width 0.8) (layer "F.Cu") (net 3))
 (segment (start 119.5 86.5) (end 119.5 82.42) (width 0.8) (layer "F.Cu") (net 3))
 (segment (start 126.5 82.42) (end 141.42 82.42) (width 0.8) (layer "F.Cu") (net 3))
 (segment (start 113.5 77) (end 113.5 81.082) (width 0.8) (layer "F.Cu") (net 3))
 (segment (start 114.838 82.42) (end 123.58 82.42) (width 0.8) (layer "F.Cu") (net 3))
 (segment (start 115.54 90) (end 119.5 90) (width 0.8) (layer "F.Cu") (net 5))
 (segment (start 126.5 92.58) (end 148.58 92.58) (width 0.8) (layer "F.Cu") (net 5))
 (segment (start 148.58 92.58) (end 158.04 102.04) (width 0.8) (layer "F.Cu") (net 5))
 (segment (start 119.5 90) (end 122.08 92.58) (width 0.8) (layer "F.Cu") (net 5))
 (segment (start 115.5 90.04) (end 115.54 90) (width 0.8) (layer "F.Cu") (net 5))
 (segment (start 122.08 92.58) (end 126.5 92.58) (width 0.8) (layer "F.Cu") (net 5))
 (segment (start 158.04 102.04) (end 158.04 105) (width 0.8) (layer "F.Cu") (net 5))
 (segment (start 117.09 69.91) (end 119 68) (width 0.8) (layer "F.Cu") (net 6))
 (segment (start 119 68) (end 119 59.86) (width 0.8) (layer "F.Cu") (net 6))
 (segment (start 115.5 69.91) (end 117.09 69.91) (width 0.8) (layer "F.Cu") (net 6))
 (segment (start 119 59.86) (end 115.88 56.74) (width 0.8) (layer "F.Cu") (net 6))
 (segment (start 153.5 80.905) (end 152.96 81.445) (width 0.8) (layer "F.Cu") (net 1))
 (segment (start 177.5 76.5) (end 165.5 76.5) (width 0.8) (layer "F.Cu") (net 1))
 (segment (start 163 79) (end 153.355 79) (width 0.8) (layer "F.Cu") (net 1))
 (segment (start 152.96 79.395) (end 152.96 81.445) (width 0.8) (layer "F.Cu") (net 1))
 (segment (start 153.355 79) (end 152.96 79.395) (width 0.8) (layer "F.Cu") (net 1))
 (segment (start 165.5 76.5) (end 163 79) (width 0.8) (layer "F.Cu") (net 1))
 (segment (start 133.46 54) (end 115.5 54) (width 0.8) (layer "F.Cu") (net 2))
 (segment (start 112 57.5) (end 112 65) (width 0.8) (layer "F.Cu") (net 2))
 (segment (start 136 54) (end 133.46 54) (width 0.8) (layer "F.Cu") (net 2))
 (segment (start 146.5 63) (end 149.5 60) (width 0.8) (layer "F.Cu") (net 2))
 (segment (start 136.2 56.74) (end 138.74 56.74) (width 0.8) (layer "F.Cu") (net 2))
 (segment (start 112 74.5) (end 112 84) (width 0.8) (layer "F.Cu") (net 2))
 (segment (start 115.5 74.5) (end 112 74.5) (width 0.8) (layer "F.Cu") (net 2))
 (segment (start 112 91) (end 122.5 101.5) (width 0.8) (layer "F.Cu") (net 2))
 (segment (start 112.17 64.83) (end 112 65) (width 0.8) (layer "F.Cu") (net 2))
 (segment (start 155.5 81.445) (end 155.5 85) (width 0.8) (layer "F.Cu") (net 2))
 (segment (start 154 86.5) (end 149.5 86.5) (width 0.8) (layer "F.Cu") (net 2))
 (segment (start 156 58) (end 156 56) (width 0.8) (layer "F.Cu") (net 2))
 (segment (start 162 86) (end 168 86) (width 0.8) (layer "F.Cu") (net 2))
 (segment (start 136.2 56.74) (end 136.2 54.2) (width 0.8) (layer "F.Cu") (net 2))
 (segment (start 115.5 84.96) (end 112.04 84.96) (width 0.8) (layer "F.Cu") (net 2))
 (segment (start 149.5 60) (end 154 60) (width 0.8) (layer "F.Cu") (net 2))
 (segment (start 136.2 54.2) (end 136 54) (width 0.8) (layer "F.Cu") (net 2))
 (segment (start 150.5 101.5) (end 152.96 103.96) (width 0.8) (layer "F.Cu") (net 2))
 (segment (start 146.5 83.5) (end 146.5 63) (width 0.8) (layer "F.Cu") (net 2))
 (segment (start 172 100.5) (end 165.5 107) (width 0.8) (layer "F.Cu") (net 2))
 (segment (start 155.5 85) (end 154 86.5) (width 0.8) (layer "F.Cu") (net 2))
 (segment (start 154.48 107) (end 152.96 105.48) (width 0.8) (layer "F.Cu") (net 2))
 (segment (start 172 86) (end 172 100.5) (width 0.8) (layer "F.Cu") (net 2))
 (segment (start 177.5 80.5) (end 172 86) (width 0.8) (layer "F.Cu") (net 2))
 (segment (start 154 54) (end 136 54) (width 0.8) (layer "F.Cu") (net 2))
 (segment (start 168 79) (end 168 86) (width 0.8) (layer "F.Cu") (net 2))
 (segment (start 115.5 54) (end 112 57.5) (width 0.8) (layer "F.Cu") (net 2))
 (segment (start 168 86) (end 172 86) (width 0.8) (layer "F.Cu") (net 2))
 (segment (start 115.5 64.83) (end 112.17 64.83) (width 0.8) (layer "F.Cu") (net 2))
 (segment (start 152.96 103.96) (end 152.96 105) (width 0.8) (layer "F.Cu") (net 2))
 (segment (start 172 86) (end 172 86.5) (width 0.8) (layer "F.Cu") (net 2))
 (segment (start 122.5 101.5) (end 150.5 101.5) (width 0.8) (layer "F.Cu") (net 2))
 (segment (start 156 56) (end 154 54) (width 0.8) (layer "F.Cu") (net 2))
 (segment (start 165.5 107) (end 154.48 107) (width 0.8) (layer "F.Cu") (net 2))
 (segment (start 112 74.5) (end 112 65) (width 0.8) (layer "F.Cu") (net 2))
 (segment (start 112.04 84.96) (end 112 85) (width 0.8) (layer "F.Cu") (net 2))
 (segment (start 152.96 105.48) (end 152.96 105) (width 0.8) (layer "F.Cu") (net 2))
 (segment (start 154 60) (end 156 58) (width 0.8) (layer "F.Cu") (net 2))
 (segment (start 112 84) (end 112 85) (width 0.8) (layer "F.Cu") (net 2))
 (segment (start 112.17 84.17) (end 112 84) (width 0.8) (layer "F.Cu") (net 2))
 (segment (start 149.5 86.5) (end 146.5 83.5) (width 0.8) (layer "F.Cu") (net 2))
 (segment (start 177.5 79.04) (end 177.5 80.5) (width 0.8) (layer "F.Cu") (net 2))
 (segment (start 112 85) (end 112 91) (width 0.8) (layer "F.Cu") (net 2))
 (segment (start 128.92 79.08) (end 131.5 76.5) (width 0.8) (layer "F.Cu") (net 4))
 (segment (start 131.5 59.66) (end 128.58 56.74) (width 0.8) (layer "F.Cu") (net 4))
 (segment (start 115.5 79.58) (end 126 79.58) (width 0.8) (layer "F.Cu") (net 4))
 (segment (start 126 79.58) (end 126.5 79.08) (width 0.8) (layer "F.Cu") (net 4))
 (segment (start 131.5 76.5) (end 131.5 59.66) (width 0.8) (layer "F.Cu") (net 4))
 (segment (start 126.5 79.08) (end 128.92 79.08) (width 0.8) (layer "F.Cu") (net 4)))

